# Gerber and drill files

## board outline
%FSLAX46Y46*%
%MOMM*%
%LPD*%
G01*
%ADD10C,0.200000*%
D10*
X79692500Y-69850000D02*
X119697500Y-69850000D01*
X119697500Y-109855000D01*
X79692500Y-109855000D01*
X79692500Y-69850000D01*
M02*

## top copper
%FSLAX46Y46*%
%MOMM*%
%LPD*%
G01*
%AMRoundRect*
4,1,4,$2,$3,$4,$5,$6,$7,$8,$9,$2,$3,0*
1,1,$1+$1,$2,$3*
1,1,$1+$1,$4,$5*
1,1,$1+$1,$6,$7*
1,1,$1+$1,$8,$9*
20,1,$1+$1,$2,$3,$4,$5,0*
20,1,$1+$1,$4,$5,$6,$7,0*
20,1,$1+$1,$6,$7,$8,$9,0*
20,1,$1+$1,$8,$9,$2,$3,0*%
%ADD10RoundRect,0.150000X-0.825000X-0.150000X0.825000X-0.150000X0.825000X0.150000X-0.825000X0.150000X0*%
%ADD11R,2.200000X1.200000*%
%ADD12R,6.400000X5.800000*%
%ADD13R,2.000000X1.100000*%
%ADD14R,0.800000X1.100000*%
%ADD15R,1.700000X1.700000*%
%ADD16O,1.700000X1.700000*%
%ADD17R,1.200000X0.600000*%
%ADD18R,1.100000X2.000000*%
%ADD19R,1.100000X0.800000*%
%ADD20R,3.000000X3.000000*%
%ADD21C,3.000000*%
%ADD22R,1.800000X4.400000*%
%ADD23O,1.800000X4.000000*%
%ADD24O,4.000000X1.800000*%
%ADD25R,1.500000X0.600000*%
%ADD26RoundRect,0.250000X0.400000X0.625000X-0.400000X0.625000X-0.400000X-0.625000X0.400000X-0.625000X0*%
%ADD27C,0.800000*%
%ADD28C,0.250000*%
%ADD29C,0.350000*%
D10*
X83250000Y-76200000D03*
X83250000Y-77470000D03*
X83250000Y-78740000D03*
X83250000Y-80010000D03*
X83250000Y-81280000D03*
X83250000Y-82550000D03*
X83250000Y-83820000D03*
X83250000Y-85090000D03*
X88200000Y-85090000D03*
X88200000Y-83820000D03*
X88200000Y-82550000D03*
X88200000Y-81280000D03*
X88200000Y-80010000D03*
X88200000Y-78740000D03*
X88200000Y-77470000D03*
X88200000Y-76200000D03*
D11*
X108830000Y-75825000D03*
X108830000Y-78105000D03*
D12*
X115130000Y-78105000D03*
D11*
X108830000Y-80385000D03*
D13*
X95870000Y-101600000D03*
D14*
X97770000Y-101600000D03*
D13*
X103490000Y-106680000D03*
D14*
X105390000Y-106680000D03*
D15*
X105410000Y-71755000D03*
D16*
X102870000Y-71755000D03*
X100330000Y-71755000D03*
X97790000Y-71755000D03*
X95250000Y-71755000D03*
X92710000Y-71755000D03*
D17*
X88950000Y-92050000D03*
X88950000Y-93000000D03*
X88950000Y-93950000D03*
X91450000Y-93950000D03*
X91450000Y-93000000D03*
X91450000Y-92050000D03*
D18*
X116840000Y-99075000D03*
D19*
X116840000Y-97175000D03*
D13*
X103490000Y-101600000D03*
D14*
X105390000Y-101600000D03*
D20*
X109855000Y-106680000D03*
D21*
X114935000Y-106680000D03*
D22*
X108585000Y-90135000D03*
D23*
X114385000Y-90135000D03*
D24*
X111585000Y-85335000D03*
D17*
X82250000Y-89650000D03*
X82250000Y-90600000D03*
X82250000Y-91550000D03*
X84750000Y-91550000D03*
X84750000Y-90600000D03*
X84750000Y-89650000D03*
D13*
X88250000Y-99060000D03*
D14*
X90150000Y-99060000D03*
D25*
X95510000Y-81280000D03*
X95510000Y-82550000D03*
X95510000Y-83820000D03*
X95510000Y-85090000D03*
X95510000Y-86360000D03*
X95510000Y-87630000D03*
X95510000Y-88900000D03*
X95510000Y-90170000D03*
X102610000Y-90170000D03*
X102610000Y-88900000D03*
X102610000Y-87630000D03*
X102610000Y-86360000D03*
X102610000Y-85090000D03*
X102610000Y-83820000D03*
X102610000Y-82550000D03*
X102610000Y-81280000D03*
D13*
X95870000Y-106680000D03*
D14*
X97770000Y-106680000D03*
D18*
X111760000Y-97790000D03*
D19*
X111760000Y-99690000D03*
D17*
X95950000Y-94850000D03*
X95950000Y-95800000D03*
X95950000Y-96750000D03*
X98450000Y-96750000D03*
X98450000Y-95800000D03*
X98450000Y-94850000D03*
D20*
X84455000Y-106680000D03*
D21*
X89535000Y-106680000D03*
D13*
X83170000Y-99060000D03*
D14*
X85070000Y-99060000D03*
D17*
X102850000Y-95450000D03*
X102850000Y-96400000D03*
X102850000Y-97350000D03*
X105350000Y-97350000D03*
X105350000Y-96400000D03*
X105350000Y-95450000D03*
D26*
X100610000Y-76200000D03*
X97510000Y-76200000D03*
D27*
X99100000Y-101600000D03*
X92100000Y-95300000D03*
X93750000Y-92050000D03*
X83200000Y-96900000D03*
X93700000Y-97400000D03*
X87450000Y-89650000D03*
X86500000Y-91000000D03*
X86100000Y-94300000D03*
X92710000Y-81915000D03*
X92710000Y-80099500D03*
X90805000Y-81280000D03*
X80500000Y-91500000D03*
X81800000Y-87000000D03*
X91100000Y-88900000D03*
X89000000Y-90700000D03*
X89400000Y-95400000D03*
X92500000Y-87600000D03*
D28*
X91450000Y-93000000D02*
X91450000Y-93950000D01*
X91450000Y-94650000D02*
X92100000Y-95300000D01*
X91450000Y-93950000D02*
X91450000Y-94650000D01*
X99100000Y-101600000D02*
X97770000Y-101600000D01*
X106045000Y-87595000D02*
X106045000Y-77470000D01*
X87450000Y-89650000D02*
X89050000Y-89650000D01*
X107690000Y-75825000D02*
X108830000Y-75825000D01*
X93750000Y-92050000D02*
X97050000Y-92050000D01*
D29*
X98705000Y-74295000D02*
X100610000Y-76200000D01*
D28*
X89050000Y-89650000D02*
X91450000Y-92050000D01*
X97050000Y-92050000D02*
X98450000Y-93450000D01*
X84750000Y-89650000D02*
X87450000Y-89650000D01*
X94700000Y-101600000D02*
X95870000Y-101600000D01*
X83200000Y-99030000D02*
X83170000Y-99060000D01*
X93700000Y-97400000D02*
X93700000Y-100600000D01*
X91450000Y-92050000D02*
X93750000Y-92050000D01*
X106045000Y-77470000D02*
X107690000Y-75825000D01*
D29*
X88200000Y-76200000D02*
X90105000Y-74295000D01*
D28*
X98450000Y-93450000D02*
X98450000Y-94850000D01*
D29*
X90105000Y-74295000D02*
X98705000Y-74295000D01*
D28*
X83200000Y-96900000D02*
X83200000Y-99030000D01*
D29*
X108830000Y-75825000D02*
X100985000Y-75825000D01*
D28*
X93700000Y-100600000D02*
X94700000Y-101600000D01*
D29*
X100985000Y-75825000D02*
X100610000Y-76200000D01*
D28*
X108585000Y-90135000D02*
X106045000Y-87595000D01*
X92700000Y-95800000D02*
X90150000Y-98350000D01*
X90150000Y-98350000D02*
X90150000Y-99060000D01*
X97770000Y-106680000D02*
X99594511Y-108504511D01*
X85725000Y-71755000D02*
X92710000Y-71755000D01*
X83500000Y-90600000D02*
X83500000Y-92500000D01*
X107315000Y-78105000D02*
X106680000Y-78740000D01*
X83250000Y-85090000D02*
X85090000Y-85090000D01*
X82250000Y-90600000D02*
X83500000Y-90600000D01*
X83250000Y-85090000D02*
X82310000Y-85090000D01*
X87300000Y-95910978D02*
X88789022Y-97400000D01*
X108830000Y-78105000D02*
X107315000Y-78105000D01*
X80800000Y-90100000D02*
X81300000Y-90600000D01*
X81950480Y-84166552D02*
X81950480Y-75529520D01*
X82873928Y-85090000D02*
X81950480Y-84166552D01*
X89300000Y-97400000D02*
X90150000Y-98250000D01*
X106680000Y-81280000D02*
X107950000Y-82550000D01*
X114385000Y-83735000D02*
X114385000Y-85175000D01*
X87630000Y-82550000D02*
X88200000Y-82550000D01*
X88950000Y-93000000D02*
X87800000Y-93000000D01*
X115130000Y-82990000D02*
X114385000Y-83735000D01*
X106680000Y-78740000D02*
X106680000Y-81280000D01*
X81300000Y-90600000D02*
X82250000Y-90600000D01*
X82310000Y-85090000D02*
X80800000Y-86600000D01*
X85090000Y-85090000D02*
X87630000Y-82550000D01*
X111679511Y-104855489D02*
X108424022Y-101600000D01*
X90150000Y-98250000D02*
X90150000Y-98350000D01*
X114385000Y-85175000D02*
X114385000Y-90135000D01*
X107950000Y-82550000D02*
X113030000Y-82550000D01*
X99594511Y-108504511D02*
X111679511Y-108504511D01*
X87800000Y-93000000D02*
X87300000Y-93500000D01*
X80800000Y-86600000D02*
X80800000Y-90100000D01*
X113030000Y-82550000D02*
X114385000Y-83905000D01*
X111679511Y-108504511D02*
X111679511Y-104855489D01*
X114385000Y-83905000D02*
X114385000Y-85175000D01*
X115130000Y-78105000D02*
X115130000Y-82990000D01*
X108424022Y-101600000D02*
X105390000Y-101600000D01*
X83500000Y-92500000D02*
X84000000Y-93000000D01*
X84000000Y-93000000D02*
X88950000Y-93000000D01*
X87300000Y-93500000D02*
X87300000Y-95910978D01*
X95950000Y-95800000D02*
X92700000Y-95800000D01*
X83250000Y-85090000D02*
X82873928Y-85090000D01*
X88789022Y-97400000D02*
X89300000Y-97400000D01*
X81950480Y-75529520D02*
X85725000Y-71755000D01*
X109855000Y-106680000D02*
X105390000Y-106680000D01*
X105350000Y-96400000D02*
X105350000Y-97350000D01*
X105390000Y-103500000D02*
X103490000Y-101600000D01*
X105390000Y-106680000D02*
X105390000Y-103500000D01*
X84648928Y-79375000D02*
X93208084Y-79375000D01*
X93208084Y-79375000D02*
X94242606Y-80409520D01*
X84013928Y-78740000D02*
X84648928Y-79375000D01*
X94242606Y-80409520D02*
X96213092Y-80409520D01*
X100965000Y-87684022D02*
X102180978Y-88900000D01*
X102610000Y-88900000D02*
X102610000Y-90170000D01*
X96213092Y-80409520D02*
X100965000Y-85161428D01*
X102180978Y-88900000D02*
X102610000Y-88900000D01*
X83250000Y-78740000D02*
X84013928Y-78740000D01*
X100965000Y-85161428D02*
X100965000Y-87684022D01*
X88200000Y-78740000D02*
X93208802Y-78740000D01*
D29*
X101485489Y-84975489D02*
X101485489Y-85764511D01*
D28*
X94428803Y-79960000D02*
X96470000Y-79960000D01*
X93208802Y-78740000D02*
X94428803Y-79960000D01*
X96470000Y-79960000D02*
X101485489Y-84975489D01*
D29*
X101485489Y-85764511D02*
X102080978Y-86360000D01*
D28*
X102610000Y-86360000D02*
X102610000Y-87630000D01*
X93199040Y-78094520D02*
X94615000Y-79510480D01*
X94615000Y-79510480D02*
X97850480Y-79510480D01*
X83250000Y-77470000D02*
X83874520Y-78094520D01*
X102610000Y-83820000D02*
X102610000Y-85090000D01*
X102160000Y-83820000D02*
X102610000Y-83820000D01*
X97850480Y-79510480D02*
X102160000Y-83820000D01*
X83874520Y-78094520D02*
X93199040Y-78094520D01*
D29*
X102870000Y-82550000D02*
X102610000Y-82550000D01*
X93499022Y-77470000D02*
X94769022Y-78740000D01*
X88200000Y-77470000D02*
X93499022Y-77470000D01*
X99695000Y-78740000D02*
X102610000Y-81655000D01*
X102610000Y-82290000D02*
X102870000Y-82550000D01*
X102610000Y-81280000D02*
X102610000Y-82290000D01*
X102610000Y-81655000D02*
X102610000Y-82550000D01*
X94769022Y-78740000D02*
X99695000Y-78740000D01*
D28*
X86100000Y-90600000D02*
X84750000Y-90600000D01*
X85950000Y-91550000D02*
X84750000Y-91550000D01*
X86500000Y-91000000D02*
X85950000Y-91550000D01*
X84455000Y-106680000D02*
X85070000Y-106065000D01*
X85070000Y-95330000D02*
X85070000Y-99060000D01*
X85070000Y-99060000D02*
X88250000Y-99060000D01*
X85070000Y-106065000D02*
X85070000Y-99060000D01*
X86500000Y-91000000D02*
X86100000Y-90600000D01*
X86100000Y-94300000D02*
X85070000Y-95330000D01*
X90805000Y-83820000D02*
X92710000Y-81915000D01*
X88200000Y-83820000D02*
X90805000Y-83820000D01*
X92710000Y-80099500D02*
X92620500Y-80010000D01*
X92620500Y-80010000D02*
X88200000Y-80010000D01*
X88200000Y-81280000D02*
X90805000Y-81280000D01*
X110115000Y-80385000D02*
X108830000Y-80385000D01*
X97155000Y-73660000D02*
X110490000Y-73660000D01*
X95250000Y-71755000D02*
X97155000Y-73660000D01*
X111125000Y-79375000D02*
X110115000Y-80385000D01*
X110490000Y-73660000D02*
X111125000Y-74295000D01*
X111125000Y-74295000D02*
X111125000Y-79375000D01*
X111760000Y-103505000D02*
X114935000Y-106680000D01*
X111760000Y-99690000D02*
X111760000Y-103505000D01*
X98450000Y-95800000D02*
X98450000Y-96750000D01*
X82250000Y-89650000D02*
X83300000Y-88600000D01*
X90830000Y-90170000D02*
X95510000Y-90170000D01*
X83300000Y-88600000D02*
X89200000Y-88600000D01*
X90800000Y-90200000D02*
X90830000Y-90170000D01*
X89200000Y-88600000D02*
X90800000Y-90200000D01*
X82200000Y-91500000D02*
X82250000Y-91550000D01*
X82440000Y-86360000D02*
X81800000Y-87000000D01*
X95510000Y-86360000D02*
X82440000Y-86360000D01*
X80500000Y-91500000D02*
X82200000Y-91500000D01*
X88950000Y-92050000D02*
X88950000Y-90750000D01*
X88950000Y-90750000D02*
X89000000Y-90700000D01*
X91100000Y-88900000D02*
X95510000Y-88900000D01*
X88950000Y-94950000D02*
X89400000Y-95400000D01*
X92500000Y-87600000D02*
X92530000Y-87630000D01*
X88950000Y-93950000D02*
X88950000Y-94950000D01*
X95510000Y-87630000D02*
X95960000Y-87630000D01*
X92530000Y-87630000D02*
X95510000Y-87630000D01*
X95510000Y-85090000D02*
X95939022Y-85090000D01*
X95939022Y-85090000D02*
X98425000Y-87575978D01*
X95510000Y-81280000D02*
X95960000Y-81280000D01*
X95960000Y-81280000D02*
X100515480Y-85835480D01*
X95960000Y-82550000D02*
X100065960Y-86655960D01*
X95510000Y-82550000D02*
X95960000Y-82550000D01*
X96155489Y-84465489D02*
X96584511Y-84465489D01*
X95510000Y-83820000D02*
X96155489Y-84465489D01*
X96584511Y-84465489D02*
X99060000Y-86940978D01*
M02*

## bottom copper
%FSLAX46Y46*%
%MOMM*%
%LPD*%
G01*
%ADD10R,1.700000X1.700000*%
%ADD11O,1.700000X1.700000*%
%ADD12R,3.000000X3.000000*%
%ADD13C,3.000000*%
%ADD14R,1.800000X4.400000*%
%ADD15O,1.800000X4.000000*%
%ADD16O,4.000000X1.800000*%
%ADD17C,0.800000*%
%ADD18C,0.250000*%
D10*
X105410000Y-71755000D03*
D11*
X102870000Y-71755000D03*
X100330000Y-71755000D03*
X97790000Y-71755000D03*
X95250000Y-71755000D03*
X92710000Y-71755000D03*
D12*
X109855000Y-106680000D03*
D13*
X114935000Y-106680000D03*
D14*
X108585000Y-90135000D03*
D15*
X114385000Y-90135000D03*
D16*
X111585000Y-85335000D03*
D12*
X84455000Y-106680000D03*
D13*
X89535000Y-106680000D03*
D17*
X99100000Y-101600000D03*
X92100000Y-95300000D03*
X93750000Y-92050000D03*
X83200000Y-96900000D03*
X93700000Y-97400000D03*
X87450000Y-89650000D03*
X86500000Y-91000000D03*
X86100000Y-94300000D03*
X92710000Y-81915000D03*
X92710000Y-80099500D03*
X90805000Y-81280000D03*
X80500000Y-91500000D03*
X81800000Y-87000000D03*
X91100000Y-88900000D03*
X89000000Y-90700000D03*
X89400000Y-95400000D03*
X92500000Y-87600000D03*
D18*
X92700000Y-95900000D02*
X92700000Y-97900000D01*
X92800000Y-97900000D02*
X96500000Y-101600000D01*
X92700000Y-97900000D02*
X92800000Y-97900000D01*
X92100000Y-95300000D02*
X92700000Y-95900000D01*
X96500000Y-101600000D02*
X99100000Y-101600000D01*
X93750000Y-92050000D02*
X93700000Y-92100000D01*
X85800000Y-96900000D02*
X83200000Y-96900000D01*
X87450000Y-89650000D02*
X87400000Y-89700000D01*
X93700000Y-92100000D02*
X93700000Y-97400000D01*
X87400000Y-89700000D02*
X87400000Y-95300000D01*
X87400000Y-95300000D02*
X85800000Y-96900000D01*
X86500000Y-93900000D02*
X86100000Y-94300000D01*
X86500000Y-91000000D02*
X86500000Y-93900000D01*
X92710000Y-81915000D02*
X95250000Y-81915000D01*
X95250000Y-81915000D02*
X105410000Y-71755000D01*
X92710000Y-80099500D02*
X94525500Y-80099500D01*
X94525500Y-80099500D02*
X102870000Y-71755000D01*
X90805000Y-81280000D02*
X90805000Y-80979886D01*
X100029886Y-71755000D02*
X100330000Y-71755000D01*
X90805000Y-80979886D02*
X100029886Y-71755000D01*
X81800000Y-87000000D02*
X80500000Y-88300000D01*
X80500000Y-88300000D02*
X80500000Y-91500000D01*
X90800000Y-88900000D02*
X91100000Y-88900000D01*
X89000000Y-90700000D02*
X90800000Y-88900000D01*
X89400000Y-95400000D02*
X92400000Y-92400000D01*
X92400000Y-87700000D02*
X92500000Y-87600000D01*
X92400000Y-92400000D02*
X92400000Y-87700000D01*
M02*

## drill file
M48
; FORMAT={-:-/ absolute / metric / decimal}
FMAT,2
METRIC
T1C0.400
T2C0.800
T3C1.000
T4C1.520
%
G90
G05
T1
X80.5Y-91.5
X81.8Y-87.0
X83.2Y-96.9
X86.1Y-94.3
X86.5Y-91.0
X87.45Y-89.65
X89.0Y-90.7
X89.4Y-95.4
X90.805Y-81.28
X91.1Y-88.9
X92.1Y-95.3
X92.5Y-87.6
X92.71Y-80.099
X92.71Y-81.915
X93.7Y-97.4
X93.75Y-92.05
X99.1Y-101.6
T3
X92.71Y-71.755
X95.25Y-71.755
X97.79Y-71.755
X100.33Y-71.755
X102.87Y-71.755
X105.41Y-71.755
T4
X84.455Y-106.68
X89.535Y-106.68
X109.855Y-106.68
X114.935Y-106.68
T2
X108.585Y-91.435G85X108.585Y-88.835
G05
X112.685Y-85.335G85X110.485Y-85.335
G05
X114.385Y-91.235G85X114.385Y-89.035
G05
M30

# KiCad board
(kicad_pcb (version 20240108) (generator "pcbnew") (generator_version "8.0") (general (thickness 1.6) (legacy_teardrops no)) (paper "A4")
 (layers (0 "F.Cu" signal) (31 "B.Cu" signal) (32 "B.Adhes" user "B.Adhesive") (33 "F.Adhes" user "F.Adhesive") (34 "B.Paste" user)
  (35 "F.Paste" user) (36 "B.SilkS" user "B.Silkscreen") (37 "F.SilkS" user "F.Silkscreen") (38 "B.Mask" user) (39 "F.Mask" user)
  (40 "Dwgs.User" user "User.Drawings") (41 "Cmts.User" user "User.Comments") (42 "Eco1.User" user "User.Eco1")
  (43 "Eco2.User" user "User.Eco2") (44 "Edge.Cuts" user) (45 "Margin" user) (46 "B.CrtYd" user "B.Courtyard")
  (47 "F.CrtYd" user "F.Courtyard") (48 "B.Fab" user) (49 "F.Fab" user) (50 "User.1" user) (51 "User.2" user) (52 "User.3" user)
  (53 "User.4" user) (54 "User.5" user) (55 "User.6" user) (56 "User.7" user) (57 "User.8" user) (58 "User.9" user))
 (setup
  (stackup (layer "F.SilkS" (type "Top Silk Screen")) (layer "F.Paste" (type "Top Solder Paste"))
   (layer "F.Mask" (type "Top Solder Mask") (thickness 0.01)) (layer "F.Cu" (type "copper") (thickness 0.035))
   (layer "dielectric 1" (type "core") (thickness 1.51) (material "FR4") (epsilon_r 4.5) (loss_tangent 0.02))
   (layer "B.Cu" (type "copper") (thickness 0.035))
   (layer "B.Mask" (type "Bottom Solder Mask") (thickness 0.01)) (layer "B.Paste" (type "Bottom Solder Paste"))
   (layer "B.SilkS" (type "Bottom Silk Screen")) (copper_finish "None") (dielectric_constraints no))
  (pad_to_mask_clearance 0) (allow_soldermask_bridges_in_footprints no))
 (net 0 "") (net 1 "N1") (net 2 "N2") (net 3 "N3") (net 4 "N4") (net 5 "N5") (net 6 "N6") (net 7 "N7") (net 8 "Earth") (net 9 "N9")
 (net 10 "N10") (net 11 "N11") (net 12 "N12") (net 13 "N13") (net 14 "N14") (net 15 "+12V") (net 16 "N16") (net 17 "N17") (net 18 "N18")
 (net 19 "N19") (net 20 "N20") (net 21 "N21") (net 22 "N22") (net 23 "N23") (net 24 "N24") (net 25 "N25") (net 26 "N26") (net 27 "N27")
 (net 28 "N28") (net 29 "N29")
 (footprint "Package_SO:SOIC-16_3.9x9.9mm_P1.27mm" (layer "F.Cu") (at 85.725 80.645)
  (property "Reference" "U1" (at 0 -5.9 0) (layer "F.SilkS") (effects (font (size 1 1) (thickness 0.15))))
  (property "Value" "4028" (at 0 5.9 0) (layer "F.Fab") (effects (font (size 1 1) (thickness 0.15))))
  (pad "1" smd roundrect (at -2.475 -4.445) (size 1.95 0.6) (layers "F.Cu" "F.Paste" "F.Mask") (roundrect_rratio 0.25) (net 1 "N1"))
  (pad "2" smd roundrect (at -2.475 -3.175) (size 1.95 0.6) (layers "F.Cu" "F.Paste" "F.Mask") (roundrect_rratio 0.25) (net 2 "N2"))
  (pad "3" smd roundrect (at -2.475 -1.905) (size 1.95 0.6) (layers "F.Cu" "F.Paste" "F.Mask") (roundrect_rratio 0.25) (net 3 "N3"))
  (pad "4" smd roundrect (at -2.475 -0.635) (size 1.95 0.6) (layers "F.Cu" "F.Paste" "F.Mask") (roundrect_rratio 0.25) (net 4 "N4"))
  (pad "5" smd roundrect (at -2.475 0.635) (size 1.95 0.6) (layers "F.Cu" "F.Paste" "F.Mask") (roundrect_rratio 0.25) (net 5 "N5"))
  (pad "6" smd roundrect (at -2.475 1.905) (size 1.95 0.6) (layers "F.Cu" "F.Paste" "F.Mask") (roundrect_rratio 0.25) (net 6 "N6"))
  (pad "7" smd roundrect (at -2.475 3.175) (size 1.95 0.6) (layers "F.Cu" "F.Paste" "F.Mask") (roundrect_rratio 0.25) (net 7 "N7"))
  (pad "8" smd roundrect (at -2.475 4.445) (size 1.95 0.6) (layers "F.Cu" "F.Paste" "F.Mask") (roundrect_rratio 0.25) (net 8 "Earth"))
  (pad "9" smd roundrect (at 2.475 4.445) (size 1.95 0.6) (layers "F.Cu" "F.Paste" "F.Mask") (roundrect_rratio 0.25) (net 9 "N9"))
  (pad "10" smd roundrect (at 2.475 3.175) (size 1.95 0.6) (layers "F.Cu" "F.Paste" "F.Mask") (roundrect_rratio 0.25) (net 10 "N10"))
  (pad "11" smd roundrect (at 2.475 1.905) (size 1.95 0.6) (layers "F.Cu" "F.Paste" "F.Mask") (roundrect_rratio 0.25) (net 8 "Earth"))
  (pad "12" smd roundrect (at 2.475 0.635) (size 1.95 0.6) (layers "F.Cu" "F.Paste" "F.Mask") (roundrect_rratio 0.25) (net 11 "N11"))
  (pad "13" smd roundrect (at 2.475 -0.635) (size 1.95 0.6) (layers "F.Cu" "F.Paste" "F.Mask") (roundrect_rratio 0.25) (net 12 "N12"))
  (pad "14" smd roundrect (at 2.475 -1.905) (size 1.95 0.6) (layers "F.Cu" "F.Paste" "F.Mask") (roundrect_rratio 0.25) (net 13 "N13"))
  (pad "15" smd roundrect (at 2.475 -3.175) (size 1.95 0.6) (layers "F.Cu" "F.Paste" "F.Mask") (roundrect_rratio 0.25) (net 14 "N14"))
  (pad "16" smd roundrect (at 2.475 -4.445) (size 1.95 0.6) (layers "F.Cu" "F.Paste" "F.Mask") (roundrect_rratio 0.25) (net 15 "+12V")))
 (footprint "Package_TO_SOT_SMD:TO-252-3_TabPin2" (layer "F.Cu") (at 113.03 78.105)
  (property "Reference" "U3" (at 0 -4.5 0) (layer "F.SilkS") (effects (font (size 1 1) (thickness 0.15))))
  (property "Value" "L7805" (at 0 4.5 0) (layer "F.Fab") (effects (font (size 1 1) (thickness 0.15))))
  (pad "" smd rect (at 0.425 -1.525) (size 3.05 2.75) (layers "F.Paste"))
  (pad "" smd rect (at 0.425 1.525) (size 3.05 2.75) (layers "F.Paste"))
  (pad "" smd rect (at 3.775 -1.525) (size 3.05 2.75) (layers "F.Paste"))
  (pad "" smd rect (at 3.775 1.525) (size 3.05 2.75) (layers "F.Paste"))
  (pad "1" smd rect (at -4.2 -2.28) (size 2.2 1.2) (layers "F.Cu" "F.Paste" "F.Mask") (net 15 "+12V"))
  (pad "2" smd rect (at -4.2 0) (size 2.2 1.2) (layers "F.Cu" "F.Paste" "F.Mask") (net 8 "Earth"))
  (pad "2" smd rect (at 2.1 0) (size 6.4 5.8) (layers "F.Cu" "F.Mask") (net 8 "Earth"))
  (pad "3" smd rect (at -4.2 2.28) (size 2.2 1.2) (layers "F.Cu" "F.Paste" "F.Mask") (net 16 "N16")))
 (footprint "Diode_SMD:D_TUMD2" (layer "F.Cu") (at 96.52 101.6)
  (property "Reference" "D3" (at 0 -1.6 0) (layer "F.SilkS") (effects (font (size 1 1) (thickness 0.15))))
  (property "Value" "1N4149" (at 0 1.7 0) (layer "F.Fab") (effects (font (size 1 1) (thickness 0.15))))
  (pad "1" smd rect (at -0.65 0 180) (size 2 1.1) (layers "F.Cu" "F.Paste" "F.Mask") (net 15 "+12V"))
  (pad "2" smd rect (at 1.25 0 180) (size 0.8 1.1) (layers "F.Cu" "F.Paste" "F.Mask") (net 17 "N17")))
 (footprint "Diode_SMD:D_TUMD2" (layer "F.Cu") (at 104.14 106.68)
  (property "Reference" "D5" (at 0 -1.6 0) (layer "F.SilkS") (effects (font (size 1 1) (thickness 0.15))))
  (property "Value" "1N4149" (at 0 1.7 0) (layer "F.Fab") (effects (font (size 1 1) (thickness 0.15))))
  (pad "1" smd rect (at -0.65 0 180) (size 2 1.1) (layers "F.Cu" "F.Paste" "F.Mask") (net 15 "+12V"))
  (pad "2" smd rect (at 1.25 0 180) (size 0.8 1.1) (layers "F.Cu" "F.Paste" "F.Mask") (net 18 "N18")))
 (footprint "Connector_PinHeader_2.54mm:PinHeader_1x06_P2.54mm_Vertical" (layer "F.Cu") (at 105.41 71.755 -90)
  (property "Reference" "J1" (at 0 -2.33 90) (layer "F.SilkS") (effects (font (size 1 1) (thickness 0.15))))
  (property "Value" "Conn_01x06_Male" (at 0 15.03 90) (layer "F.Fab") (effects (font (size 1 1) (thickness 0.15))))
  (pad "1" thru_hole rect (at 0 0 270) (size 1.7 1.7) (drill 1) (layers "*.Cu" "*.Mask") (remove_unused_layers no) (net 10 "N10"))
  (pad "2" thru_hole oval (at 0 2.54 270) (size 1.7 1.7) (drill 1) (layers "*.Cu" "*.Mask") (remove_unused_layers no) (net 12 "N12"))
  (pad "3" thru_hole oval (at 0 5.08 270) (size 1.7 1.7) (drill 1) (layers "*.Cu" "*.Mask") (remove_unused_layers no) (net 11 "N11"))
  (pad "4" thru_hole oval (at 0 7.62 270) (size 1.7 1.7) (drill 1) (layers "*.Cu" "*.Mask") (remove_unused_layers no) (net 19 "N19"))
  (pad "5" thru_hole oval (at 0 10.16 270) (size 1.7 1.7) (drill 1) (layers "*.Cu" "*.Mask") (remove_unused_layers no) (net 16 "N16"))
  (pad "6" thru_hole oval (at 0 12.7 270) (size 1.7 1.7) (drill 1) (layers "*.Cu" "*.Mask") (remove_unused_layers no) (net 8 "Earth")))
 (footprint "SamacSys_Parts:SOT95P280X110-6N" (layer "F.Cu") (at 90.2 93)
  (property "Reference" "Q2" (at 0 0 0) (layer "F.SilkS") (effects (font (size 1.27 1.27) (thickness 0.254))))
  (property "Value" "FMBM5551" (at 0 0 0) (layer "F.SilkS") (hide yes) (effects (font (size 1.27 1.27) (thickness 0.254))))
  (pad "1" smd rect (at -1.25 -0.95 90) (size 0.6 1.2) (layers "F.Cu" "F.Paste" "F.Mask") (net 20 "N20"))
  (pad "2" smd rect (at -1.25 0 90) (size 0.6 1.2) (layers "F.Cu" "F.Paste" "F.Mask") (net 8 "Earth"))
  (pad "3" smd rect (at -1.25 0.95 90) (size 0.6 1.2) (layers "F.Cu" "F.Paste" "F.Mask") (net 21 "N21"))
  (pad "4" smd rect (at 1.25 0.95 90) (size 0.6 1.2) (layers "F.Cu" "F.Paste" "F.Mask") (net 17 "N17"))
  (pad "5" smd rect (at 1.25 0 90) (size 0.6 1.2) (layers "F.Cu" "F.Paste" "F.Mask") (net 17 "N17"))
  (pad "6" smd rect (at 1.25 -0.95 90) (size 0.6 1.2) (layers "F.Cu" "F.Paste" "F.Mask") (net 15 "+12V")))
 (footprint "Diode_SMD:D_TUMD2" (layer "F.Cu") (at 116.84 98.425 90)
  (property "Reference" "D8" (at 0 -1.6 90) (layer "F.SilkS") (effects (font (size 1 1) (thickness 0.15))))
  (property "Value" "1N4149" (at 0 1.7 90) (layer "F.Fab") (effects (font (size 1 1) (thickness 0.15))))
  (pad "1" smd rect (at -0.65 0 270) (size 2 1.1) (layers "F.Cu" "F.Paste" "F.Mask") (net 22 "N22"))
  (pad "2" smd rect (at 1.25 0 270) (size 0.8 1.1) (layers "F.Cu" "F.Paste" "F.Mask") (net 8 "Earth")))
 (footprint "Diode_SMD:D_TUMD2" (layer "F.Cu") (at 104.14 101.6)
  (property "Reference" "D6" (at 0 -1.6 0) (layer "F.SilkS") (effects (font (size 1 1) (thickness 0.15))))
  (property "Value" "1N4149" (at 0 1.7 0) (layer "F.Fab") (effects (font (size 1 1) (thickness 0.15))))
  (pad "1" smd rect (at -0.65 0 180) (size 2 1.1) (layers "F.Cu" "F.Paste" "F.Mask") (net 18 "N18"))
  (pad "2" smd rect (at 1.25 0 180) (size 0.8 1.1) (layers "F.Cu" "F.Paste" "F.Mask") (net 8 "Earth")))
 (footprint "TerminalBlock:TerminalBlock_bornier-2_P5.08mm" (layer "F.Cu") (at 109.855 106.68)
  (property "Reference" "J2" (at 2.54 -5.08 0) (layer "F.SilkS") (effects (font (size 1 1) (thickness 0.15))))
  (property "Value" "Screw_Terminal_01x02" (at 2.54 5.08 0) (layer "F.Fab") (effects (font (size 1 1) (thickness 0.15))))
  (pad "1" thru_hole rect (at 0 0) (size 3 3) (drill 1.52) (layers "*.Cu" "*.Mask") (remove_unused_layers no) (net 18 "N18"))
  (pad "2" thru_hole circle (at 5.08 0) (size 3 3) (drill 1.52) (layers "*.Cu" "*.Mask") (remove_unused_layers no) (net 22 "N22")))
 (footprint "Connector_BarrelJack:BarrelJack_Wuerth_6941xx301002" (layer "F.Cu") (at 108.585 90.135 90)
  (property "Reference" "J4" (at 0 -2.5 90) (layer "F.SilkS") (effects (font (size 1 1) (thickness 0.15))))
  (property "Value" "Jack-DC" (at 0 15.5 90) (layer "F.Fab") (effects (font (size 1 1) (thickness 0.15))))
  (pad "1" thru_hole rect (at 0 0 90) (size 4.4 1.8) (drill oval 3.4 0.8) (layers "*.Cu" "*.Mask") (remove_unused_layers no) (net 15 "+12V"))
  (pad "2" thru_hole oval (at 0 5.8 90) (size 4 1.8) (drill oval 3 0.8) (layers "*.Cu" "*.Mask") (remove_unused_layers no) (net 8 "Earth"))
  (pad "3" thru_hole oval (at 4.8 3 180) (size 4 1.8) (drill oval 3 0.8) (layers "*.Cu" "*.Mask") (remove_unused_layers no)))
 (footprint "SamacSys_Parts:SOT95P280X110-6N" (layer "F.Cu") (at 83.5 90.6)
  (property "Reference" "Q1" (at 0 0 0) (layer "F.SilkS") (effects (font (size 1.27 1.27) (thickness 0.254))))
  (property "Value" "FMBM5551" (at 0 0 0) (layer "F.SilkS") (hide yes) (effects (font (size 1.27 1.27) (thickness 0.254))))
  (pad "1" smd rect (at -1.25 -0.95 90) (size 0.6 1.2) (layers "F.Cu" "F.Paste" "F.Mask") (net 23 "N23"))
  (pad "2" smd rect (at -1.25 0 90) (size 0.6 1.2) (layers "F.Cu" "F.Paste" "F.Mask") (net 8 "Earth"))
  (pad "3" smd rect (at -1.25 0.95 90) (size 0.6 1.2) (layers "F.Cu" "F.Paste" "F.Mask") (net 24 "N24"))
  (pad "4" smd rect (at 1.25 0.95 90) (size 0.6 1.2) (layers "F.Cu" "F.Paste" "F.Mask") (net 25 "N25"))
  (pad "5" smd rect (at 1.25 0 90) (size 0.6 1.2) (layers "F.Cu" "F.Paste" "F.Mask") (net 25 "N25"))
  (pad "6" smd rect (at 1.25 -0.95 90) (size 0.6 1.2) (layers "F.Cu" "F.Paste" "F.Mask") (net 15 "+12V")))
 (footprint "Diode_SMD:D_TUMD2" (layer "F.Cu") (at 88.9 99.06)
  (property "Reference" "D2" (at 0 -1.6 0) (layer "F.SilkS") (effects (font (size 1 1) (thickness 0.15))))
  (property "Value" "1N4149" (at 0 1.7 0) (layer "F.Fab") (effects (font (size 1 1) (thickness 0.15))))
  (pad "1" smd rect (at -0.65 0 180) (size 2 1.1) (layers "F.Cu" "F.Paste" "F.Mask") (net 25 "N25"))
  (pad "2" smd rect (at 1.25 0 180) (size 0.8 1.1) (layers "F.Cu" "F.Paste" "F.Mask") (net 8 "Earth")))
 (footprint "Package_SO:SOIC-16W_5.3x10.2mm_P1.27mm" (layer "F.Cu") (at 99.06 85.725)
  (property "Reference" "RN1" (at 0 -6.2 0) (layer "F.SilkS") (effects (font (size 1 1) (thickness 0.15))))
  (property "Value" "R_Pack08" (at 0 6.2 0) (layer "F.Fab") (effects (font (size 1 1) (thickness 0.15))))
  (pad "1" smd rect (at -3.55 -4.445) (size 1.5 0.6) (layers "F.Cu" "F.Paste" "F.Mask") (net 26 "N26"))
  (pad "2" smd rect (at -3.55 -3.175) (size 1.5 0.6) (layers "F.Cu" "F.Paste" "F.Mask") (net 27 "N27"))
  (pad "3" smd rect (at -3.55 -1.905) (size 1.5 0.6) (layers "F.Cu" "F.Paste" "F.Mask") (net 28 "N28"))
  (pad "4" smd rect (at -3.55 -0.635) (size 1.5 0.6) (layers "F.Cu" "F.Paste" "F.Mask") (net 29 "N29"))
  (pad "5" smd rect (at -3.55 0.635) (size 1.5 0.6) (layers "F.Cu" "F.Paste" "F.Mask") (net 24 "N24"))
  (pad "6" smd rect (at -3.55 1.905) (size 1.5 0.6) (layers "F.Cu" "F.Paste" "F.Mask") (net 21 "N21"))
  (pad "7" smd rect (at -3.55 3.175) (size 1.5 0.6) (layers "F.Cu" "F.Paste" "F.Mask") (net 20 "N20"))
  (pad "8" smd rect (at -3.55 4.445) (size 1.5 0.6) (layers "F.Cu" "F.Paste" "F.Mask") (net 23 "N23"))
  (pad "9" smd rect (at 3.55 4.445) (size 1.5 0.6) (layers "F.Cu" "F.Paste" "F.Mask") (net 3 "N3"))
  (pad "10" smd rect (at 3.55 3.175) (size 1.5 0.6) (layers "F.Cu" "F.Paste" "F.Mask") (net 3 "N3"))
  (pad "11" smd rect (at 3.55 1.905) (size 1.5 0.6) (layers "F.Cu" "F.Paste" "F.Mask") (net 13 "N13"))
  (pad "12" smd rect (at 3.55 0.635) (size 1.5 0.6) (layers "F.Cu" "F.Paste" "F.Mask") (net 13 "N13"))
  (pad "13" smd rect (at 3.55 -0.635) (size 1.5 0.6) (layers "F.Cu" "F.Paste" "F.Mask") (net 2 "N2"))
  (pad "14" smd rect (at 3.55 -1.905) (size 1.5 0.6) (layers "F.Cu" "F.Paste" "F.Mask") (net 2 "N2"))
  (pad "15" smd rect (at 3.55 -3.175) (size 1.5 0.6) (layers "F.Cu" "F.Paste" "F.Mask") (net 14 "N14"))
  (pad "16" smd rect (at 3.55 -4.445) (size 1.5 0.6) (layers "F.Cu" "F.Paste" "F.Mask") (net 14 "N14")))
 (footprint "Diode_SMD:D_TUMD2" (layer "F.Cu") (at 96.52 106.68)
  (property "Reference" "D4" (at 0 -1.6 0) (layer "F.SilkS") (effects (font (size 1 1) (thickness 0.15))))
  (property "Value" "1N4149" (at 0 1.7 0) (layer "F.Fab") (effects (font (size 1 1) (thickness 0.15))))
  (pad "1" smd rect (at -0.65 0 180) (size 2 1.1) (layers "F.Cu" "F.Paste" "F.Mask") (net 17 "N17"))
  (pad "2" smd rect (at 1.25 0 180) (size 0.8 1.1) (layers "F.Cu" "F.Paste" "F.Mask") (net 8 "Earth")))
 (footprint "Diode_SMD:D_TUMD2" (layer "F.Cu") (at 111.76 98.44 -90)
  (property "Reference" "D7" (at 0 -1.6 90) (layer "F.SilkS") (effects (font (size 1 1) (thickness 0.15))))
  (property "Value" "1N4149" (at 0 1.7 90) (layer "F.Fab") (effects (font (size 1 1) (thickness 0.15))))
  (pad "1" smd rect (at -0.65 0 90) (size 2 1.1) (layers "F.Cu" "F.Paste" "F.Mask") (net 15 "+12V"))
  (pad "2" smd rect (at 1.25 0 90) (size 0.8 1.1) (layers "F.Cu" "F.Paste" "F.Mask") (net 22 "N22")))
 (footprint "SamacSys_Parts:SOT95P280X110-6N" (layer "F.Cu") (at 97.2 95.8)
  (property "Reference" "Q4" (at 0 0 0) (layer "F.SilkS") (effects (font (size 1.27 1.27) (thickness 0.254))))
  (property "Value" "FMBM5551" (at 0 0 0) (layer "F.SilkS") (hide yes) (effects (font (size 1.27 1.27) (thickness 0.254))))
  (pad "1" smd rect (at -1.25 -0.95 90) (size 0.6 1.2) (layers "F.Cu" "F.Paste" "F.Mask") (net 27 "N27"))
  (pad "2" smd rect (at -1.25 0 90) (size 0.6 1.2) (layers "F.Cu" "F.Paste" "F.Mask") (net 8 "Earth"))
  (pad "3" smd rect (at -1.25 0.95 90) (size 0.6 1.2) (layers "F.Cu" "F.Paste" "F.Mask") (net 28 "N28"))
  (pad "4" smd rect (at 1.25 0.95 90) (size 0.6 1.2) (layers "F.Cu" "F.Paste" "F.Mask") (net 22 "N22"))
  (pad "5" smd rect (at 1.25 0 90) (size 0.6 1.2) (layers "F.Cu" "F.Paste" "F.Mask") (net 22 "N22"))
  (pad "6" smd rect (at 1.25 -0.95 90) (size 0.6 1.2) (layers "F.Cu" "F.Paste" "F.Mask") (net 15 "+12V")))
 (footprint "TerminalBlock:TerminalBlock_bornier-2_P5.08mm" (layer "F.Cu") (at 84.455 106.68)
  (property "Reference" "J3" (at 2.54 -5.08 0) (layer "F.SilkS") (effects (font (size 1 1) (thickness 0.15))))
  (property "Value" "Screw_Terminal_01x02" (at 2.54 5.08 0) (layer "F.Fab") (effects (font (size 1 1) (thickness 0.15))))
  (pad "1" thru_hole rect (at 0 0) (size 3 3) (drill 1.52) (layers "*.Cu" "*.Mask") (remove_unused_layers no) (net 25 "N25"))
  (pad "2" thru_hole circle (at 5.08 0) (size 3 3) (drill 1.52) (layers "*.Cu" "*.Mask") (remove_unused_layers no) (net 17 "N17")))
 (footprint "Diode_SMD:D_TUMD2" (layer "F.Cu") (at 83.82 99.06)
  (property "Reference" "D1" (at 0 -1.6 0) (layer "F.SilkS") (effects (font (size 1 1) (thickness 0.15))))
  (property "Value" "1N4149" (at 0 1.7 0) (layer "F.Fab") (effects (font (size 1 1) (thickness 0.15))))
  (pad "1" smd rect (at -0.65 0 180) (size 2 1.1) (layers "F.Cu" "F.Paste" "F.Mask") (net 15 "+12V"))
  (pad "2" smd rect (at 1.25 0 180) (size 0.8 1.1) (layers "F.Cu" "F.Paste" "F.Mask") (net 25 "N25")))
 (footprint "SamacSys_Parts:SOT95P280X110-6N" (layer "F.Cu") (at 104.1 96.4)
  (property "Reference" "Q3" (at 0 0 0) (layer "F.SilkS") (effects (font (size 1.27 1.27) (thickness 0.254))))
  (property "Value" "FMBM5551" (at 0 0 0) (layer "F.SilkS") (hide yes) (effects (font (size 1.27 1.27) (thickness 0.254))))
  (pad "1" smd rect (at -1.25 -0.95 90) (size 0.6 1.2) (layers "F.Cu" "F.Paste" "F.Mask") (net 29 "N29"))
  (pad "2" smd rect (at -1.25 0 90) (size 0.6 1.2) (layers "F.Cu" "F.Paste" "F.Mask") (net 8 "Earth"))
  (pad "3" smd rect (at -1.25 0.95 90) (size 0.6 1.2) (layers "F.Cu" "F.Paste" "F.Mask") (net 26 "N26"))
  (pad "4" smd rect (at 1.25 0.95 90) (size 0.6 1.2) (layers "F.Cu" "F.Paste" "F.Mask") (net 18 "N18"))
  (pad "5" smd rect (at 1.25 0 90) (size 0.6 1.2) (layers "F.Cu" "F.Paste" "F.Mask") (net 18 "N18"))
  (pad "6" smd rect (at 1.25 -0.95 90) (size 0.6 1.2) (layers "F.Cu" "F.Paste" "F.Mask") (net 15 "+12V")))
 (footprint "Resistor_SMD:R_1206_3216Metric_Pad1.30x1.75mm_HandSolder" (layer "F.Cu") (at 99.06 76.2 180)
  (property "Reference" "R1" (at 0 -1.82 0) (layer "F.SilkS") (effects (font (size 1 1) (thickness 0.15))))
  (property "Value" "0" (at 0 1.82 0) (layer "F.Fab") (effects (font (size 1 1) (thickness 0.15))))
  (pad "1" smd roundrect (at -1.55 0 180) (size 1.3 1.75) (layers "F.Cu" "F.Paste" "F.Mask") (roundrect_rratio 0.192308) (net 15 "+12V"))
  (pad "2" smd roundrect (at 1.55 0 180) (size 1.3 1.75) (layers "F.Cu" "F.Paste" "F.Mask") (roundrect_rratio 0.192308) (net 19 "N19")))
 (gr_rect (start 79.6925 69.85) (end 119.6975 109.855) (stroke (width 0.2) (type solid)) (fill none) (layer "Edge.Cuts"))
 (segment (start 91.45 93) (end 91.45 93.95) (width 0.25) (layer "F.Cu") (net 17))
 (segment (start 91.45 94.65) (end 92.1 95.3) (width 0.25) (layer "F.Cu") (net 17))
 (segment (start 91.45 93.95) (end 91.45 94.65) (width 0.25) (layer "F.Cu") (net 17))
 (segment (start 99.1 101.6) (end 97.77 101.6) (width 0.25) (layer "F.Cu") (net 17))
 (via (at 99.1 101.6) (size 0.8) (drill 0.4) (layers "F.Cu" "B.Cu") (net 17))
 (via (at 92.1 95.3) (size 0.8) (drill 0.4) (layers "F.Cu" "B.Cu") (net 17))
 (segment (start 92.7 95.9) (end 92.7 97.9) (width 0.25) (layer "B.Cu") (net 17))
 (segment (start 92.8 97.9) (end 96.5 101.6) (width 0.25) (layer "B.Cu") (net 17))
 (segment (start 92.7 97.9) (end 92.8 97.9) (width 0.25) (layer "B.Cu") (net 17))
 (segment (start 92.1 95.3) (end 92.7 95.9) (width 0.25) (layer "B.Cu") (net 17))
 (segment (start 96.5 101.6) (end 99.1 101.6) (width 0.25) (layer "B.Cu") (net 17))
 (segment (start 106.045 87.595) (end 106.045 77.47) (width 0.25) (layer "F.Cu") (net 15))
 (segment (start 87.45 89.65) (end 89.05 89.65) (width 0.25) (layer "F.Cu") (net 15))
 (segment (start 107.69 75.825) (end 108.83 75.825) (width 0.25) (layer "F.Cu") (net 15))
 (segment (start 93.75 92.05) (end 97.05 92.05) (width 0.25) (layer "F.Cu") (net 15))
 (segment (start 98.705 74.295) (end 100.61 76.2) (width 0.35) (layer "F.Cu") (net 15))
 (segment (start 89.05 89.65) (end 91.45 92.05) (width 0.25) (layer "F.Cu") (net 15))
 (segment (start 97.05 92.05) (end 98.45 93.45) (width 0.25) (layer "F.Cu") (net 15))
 (segment (start 84.75 89.65) (end 87.45 89.65) (width 0.25) (layer "F.Cu") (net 15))
 (segment (start 94.7 101.6) (end 95.87 101.6) (width 0.25) (layer "F.Cu") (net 15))
 (segment (start 83.2 99.03) (end 83.17 99.06) (width 0.25) (layer "F.Cu") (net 15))
 (segment (start 93.7 97.4) (end 93.7 100.6) (width 0.25) (layer "F.Cu") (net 15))
 (segment (start 91.45 92.05) (end 93.75 92.05) (width 0.25) (layer "F.Cu") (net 15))
 (segment (start 106.045 77.47) (end 107.69 75.825) (width 0.25) (layer "F.Cu") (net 15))
 (segment (start 88.2 76.2) (end 90.105 74.295) (width 0.35) (layer "F.Cu") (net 15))
 (segment (start 98.45 93.45) (end 98.45 94.85) (width 0.25) (layer "F.Cu") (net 15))
 (segment (start 90.105 74.295) (end 98.705 74.295) (width 0.35) (layer "F.Cu") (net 15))
 (segment (start 83.2 96.9) (end 83.2 99.03) (width 0.25) (layer "F.Cu") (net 15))
 (segment (start 108.83 75.825) (end 100.985 75.825) (width 0.35) (layer "F.Cu") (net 15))
 (segment (start 93.7 100.6) (end 94.7 101.6) (width 0.25) (layer "F.Cu") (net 15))
 (segment (start 100.985 75.825) (end 100.61 76.2) (width 0.35) (layer "F.Cu") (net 15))
 (segment (start 108.585 90.135) (end 106.045 87.595) (width 0.25) (layer "F.Cu") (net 15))
 (via (at 93.75 92.05) (size 0.8) (drill 0.4) (layers "F.Cu" "B.Cu") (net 15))
 (via (at 83.2 96.9) (size 0.8) (drill 0.4) (layers "F.Cu" "B.Cu") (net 15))
 (via (at 93.7 97.4) (size 0.8) (drill 0.4) (layers "F.Cu" "B.Cu") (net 15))
 (via (at 87.45 89.65) (size 0.8) (drill 0.4) (layers "F.Cu" "B.Cu") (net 15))
 (segment (start 93.75 92.05) (end 93.7 92.1) (width 0.25) (layer "B.Cu") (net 15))
 (segment (start 85.8 96.9) (end 83.2 96.9) (width 0.25) (layer "B.Cu") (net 15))
 (segment (start 87.45 89.65) (end 87.4 89.7) (width 0.25) (layer "B.Cu") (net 15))
 (segment (start 93.7 92.1) (end 93.7 97.4) (width 0.25) (layer "B.Cu") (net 15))
 (segment (start 87.4 89.7) (end 87.4 95.3) (width 0.25) (layer "B.Cu") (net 15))
 (segment (start 87.4 95.3) (end 85.8 96.9) (width 0.25) (layer "B.Cu") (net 15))
 (segment (start 92.7 95.8) (end 90.15 98.35) (width 0.25) (layer "F.Cu") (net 8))
 (segment (start 90.15 98.35) (end 90.15 99.06) (width 0.25) (layer "F.Cu") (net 8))
 (segment (start 97.77 106.68) (end 99.594511 108.504511) (width 0.25) (layer "F.Cu") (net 8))
 (segment (start 85.725 71.755) (end 92.71 71.755) (width 0.25) (layer "F.Cu") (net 8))
 (segment (start 83.5 90.6) (end 83.5 92.5) (width 0.25) (layer "F.Cu") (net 8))
 (segment (start 107.315 78.105) (end 106.68 78.74) (width 0.25) (layer "F.Cu") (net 8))
 (segment (start 83.25 85.09) (end 85.09 85.09) (width 0.25) (layer "F.Cu") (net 8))
 (segment (start 82.25 90.6) (end 83.5 90.6) (width 0.25) (layer "F.Cu") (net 8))
 (segment (start 83.25 85.09) (end 82.31 85.09) (width 0.25) (layer "F.Cu") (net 8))
 (segment (start 87.3 95.910978) (end 88.789022 97.4) (width 0.25) (layer "F.Cu") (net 8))
 (segment (start 108.83 78.105) (end 107.315 78.105) (width 0.25) (layer "F.Cu") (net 8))
 (segment (start 80.8 90.1) (end 81.3 90.6) (width 0.25) (layer "F.Cu") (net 8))
 (segment (start 81.95048 84.166552) (end 81.95048 75.52952) (width 0.25) (layer "F.Cu") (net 8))
 (segment (start 82.873928 85.09) (end 81.95048 84.166552) (width 0.25) (layer "F.Cu") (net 8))
 (segment (start 89.3 97.4) (end 90.15 98.25) (width 0.25) (layer "F.Cu") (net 8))
 (segment (start 106.68 81.28) (end 107.95 82.55) (width 0.25) (layer "F.Cu") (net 8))
 (segment (start 114.385 83.735) (end 114.385 85.175) (width 0.25) (layer "F.Cu") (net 8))
 (segment (start 87.63 82.55) (end 88.2 82.55) (width 0.25) (layer "F.Cu") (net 8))
 (segment (start 88.95 93) (end 87.8 93) (width 0.25) (layer "F.Cu") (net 8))
 (segment (start 115.13 82.99) (end 114.385 83.735) (width 0.25) (layer "F.Cu") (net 8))
 (segment (start 106.68 78.74) (end 106.68 81.28) (width 0.25) (layer "F.Cu") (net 8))
 (segment (start 81.3 90.6) (end 82.25 90.6) (width 0.25) (layer "F.Cu") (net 8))
 (segment (start 82.31 85.09) (end 80.8 86.6) (width 0.25) (layer "F.Cu") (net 8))
 (segment (start 85.09 85.09) (end 87.63 82.55) (width 0.25) (layer "F.Cu") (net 8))
 (segment (start 111.679511 104.855489) (end 108.424022 101.6) (width 0.25) (layer "F.Cu") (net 8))
 (segment (start 90.15 98.25) (end 90.15 98.35) (width 0.25) (layer "F.Cu") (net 8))
 (segment (start 114.385 85.175) (end 114.385 90.135) (width 0.25) (layer "F.Cu") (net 8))
 (segment (start 107.95 82.55) (end 113.03 82.55) (width 0.25) (layer "F.Cu") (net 8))
 (segment (start 99.594511 108.504511) (end 111.679511 108.504511) (width 0.25) (layer "F.Cu") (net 8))
 (segment (start 87.8 93) (end 87.3 93.5) (width 0.25) (layer "F.Cu") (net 8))
 (segment (start 80.8 86.6) (end 80.8 90.1) (width 0.25) (layer "F.Cu") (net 8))
 (segment (start 113.03 82.55) (end 114.385 83.905) (width 0.25) (layer "F.Cu") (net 8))
 (segment (start 111.679511 108.504511) (end 111.679511 104.855489) (width 0.25) (layer "F.Cu") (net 8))
 (segment (start 114.385 83.905) (end 114.385 85.175) (width 0.25) (layer "F.Cu") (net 8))
 (segment (start 115.13 78.105) (end 115.13 82.99) (width 0.25) (layer "F.Cu") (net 8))
 (segment (start 108.424022 101.6) (end 105.39 101.6) (width 0.25) (layer "F.Cu") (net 8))
 (segment (start 83.5 92.5) (end 84 93) (width 0.25) (layer "F.Cu") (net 8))
 (segment (start 84 93) (end 88.95 93) (width 0.25) (layer "F.Cu") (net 8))
 (segment (start 87.3 93.5) (end 87.3 95.910978) (width 0.25) (layer "F.Cu") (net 8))
 (segment (start 95.95 95.8) (end 92.7 95.8) (width 0.25) (layer "F.Cu") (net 8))
 (segment (start 83.25 85.09) (end 82.873928 85.09) (width 0.25) (layer "F.Cu") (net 8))
 (segment (start 88.789022 97.4) (end 89.3 97.4) (width 0.25) (layer "F.Cu") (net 8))
 (segment (start 81.95048 75.52952) (end 85.725 71.755) (width 0.25) (layer "F.Cu") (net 8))
 (segment (start 109.855 106.68) (end 105.39 106.68) (width 0.25) (layer "F.Cu") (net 18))
 (segment (start 105.35 96.4) (end 105.35 97.35) (width 0.25) (layer "F.Cu") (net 18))
 (segment (start 105.39 103.5) (end 103.49 101.6) (width 0.25) (layer "F.Cu") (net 18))
 (segment (start 105.39 106.68) (end 105.39 103.5) (width 0.25) (layer "F.Cu") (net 18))
 (segment (start 84.648928 79.375) (end 93.208084 79.375) (width 0.25) (layer "F.Cu") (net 3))
 (segment (start 93.208084 79.375) (end 94.242606 80.40952) (width 0.25) (layer "F.Cu") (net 3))
 (segment (start 84.013928 78.74) (end 84.648928 79.375) (width 0.25) (layer "F.Cu") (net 3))
 (segment (start 94.242606 80.40952) (end 96.213092 80.40952) (width 0.25) (layer "F.Cu") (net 3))
 (segment (start 100.965 87.684022) (end 102.180978 88.9) (width 0.25) (layer "F.Cu") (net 3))
 (segment (start 102.61 88.9) (end 102.61 90.17) (width 0.25) (layer "F.Cu") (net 3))
 (segment (start 96.213092 80.40952) (end 100.965 85.161428) (width 0.25) (layer "F.Cu") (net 3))
 (segment (start 102.180978 88.9) (end 102.61 88.9) (width 0.25) (layer "F.Cu") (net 3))
 (segment (start 83.25 78.74) (end 84.013928 78.74) (width 0.25) (layer "F.Cu") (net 3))
 (segment (start 100.965 85.161428) (end 100.965 87.684022) (width 0.25) (layer "F.Cu") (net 3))
 (segment (start 88.2 78.74) (end 93.208802 78.74) (width 0.25) (layer "F.Cu") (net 13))
 (segment (start 101.485489 84.975489) (end 101.485489 85.764511) (width 0.35) (layer "F.Cu") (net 13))
 (segment (start 94.428803 79.96) (end 96.47 79.96) (width 0.25) (layer "F.Cu") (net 13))
 (segment (start 93.208802 78.74) (end 94.428803 79.96) (width 0.25) (layer "F.Cu") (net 13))
 (segment (start 96.47 79.96) (end 101.485489 84.975489) (width 0.25) (layer "F.Cu") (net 13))
 (segment (start 101.485489 85.764511) (end 102.080978 86.36) (width 0.35) (layer "F.Cu") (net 13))
 (segment (start 102.61 86.36) (end 102.61 87.63) (width 0.25) (layer "F.Cu") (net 13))
 (segment (start 93.19904 78.09452) (end 94.615 79.51048) (width 0.25) (layer "F.Cu") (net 2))
 (segment (start 94.615 79.51048) (end 97.85048 79.51048) (width 0.25) (layer "F.Cu") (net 2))
 (segment (start 83.25 77.47) (end 83.87452 78.09452) (width 0.25) (layer "F.Cu") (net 2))
 (segment (start 102.61 83.82) (end 102.61 85.09) (width 0.25) (layer "F.Cu") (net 2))
 (segment (start 102.16 83.82) (end 102.61 83.82) (width 0.25) (layer "F.Cu") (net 2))
 (segment (start 97.85048 79.51048) (end 102.16 83.82) (width 0.25) (layer "F.Cu") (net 2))
 (segment (start 83.87452 78.09452) (end 93.19904 78.09452) (width 0.25) (layer "F.Cu") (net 2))
 (segment (start 102.87 82.55) (end 102.61 82.55) (width 0.35) (layer "F.Cu") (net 14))
 (segment (start 93.499022 77.47) (end 94.769022 78.74) (width 0.35) (layer "F.Cu") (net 14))
 (segment (start 88.2 77.47) (end 93.499022 77.47) (width 0.35) (layer "F.Cu") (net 14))
 (segment (start 99.695 78.74) (end 102.61 81.655) (width 0.35) (layer "F.Cu") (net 14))
 (segment (start 102.61 82.29) (end 102.87 82.55) (width 0.35) (layer "F.Cu") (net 14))
 (segment (start 102.61 81.28) (end 102.61 82.29) (width 0.35) (layer "F.Cu") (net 14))
 (segment (start 102.61 81.655) (end 102.61 82.55) (width 0.35) (layer "F.Cu") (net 14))
 (segment (start 94.769022 78.74) (end 99.695 78.74) (width 0.35) (layer "F.Cu") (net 14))
 (segment (start 86.1 90.6) (end 84.75 90.6) (width 0.25) (layer "F.Cu") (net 25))
 (segment (start 85.95 91.55) (end 84.75 91.55) (width 0.25) (layer "F.Cu") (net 25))
 (segment (start 86.5 91) (end 85.95 91.55) (width 0.25) (layer "F.Cu") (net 25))
 (segment (start 84.455 106.68) (end 85.07 106.065) (width 0.25) (layer "F.Cu") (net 25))
 (segment (start 85.07 95.33) (end 85.07 99.06) (width 0.25) (layer "F.Cu") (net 25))
 (segment (start 85.07 99.06) (end 88.25 99.06) (width 0.25) (layer "F.Cu") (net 25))
 (segment (start 85.07 106.065) (end 85.07 99.06) (width 0.25) (layer "F.Cu") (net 25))
 (segment (start 86.5 91) (end 86.1 90.6) (width 0.25) (layer "F.Cu") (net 25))
 (segment (start 86.1 94.3) (end 85.07 95.33) (width 0.25) (layer "F.Cu") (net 25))
 (via (at 86.5 91) (size 0.8) (drill 0.4) (layers "F.Cu" "B.Cu") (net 25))
 (via (at 86.1 94.3) (size 0.8) (drill 0.4) (layers "F.Cu" "B.Cu") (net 25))
 (segment (start 86.5 93.9) (end 86.1 94.3) (width 0.25) (layer "B.Cu") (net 25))
 (segment (start 86.5 91) (end 86.5 93.9) (width 0.25) (layer "B.Cu") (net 25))
 (segment (start 90.805 83.82) (end 92.71 81.915) (width 0.25) (layer "F.Cu") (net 10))
 (segment (start 88.2 83.82) (end 90.805 83.82) (width 0.25) (layer "F.Cu") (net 10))
 (via (at 92.71 81.915) (size 0.8) (drill 0.4) (layers "F.Cu" "B.Cu") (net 10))
 (segment (start 92.71 81.915) (end 95.25 81.915) (width 0.25) (layer "B.Cu") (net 10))
 (segment (start 95.25 81.915) (end 105.41 71.755) (width 0.25) (layer "B.Cu") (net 10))
 (segment (start 92.71 80.0995) (end 92.6205 80.01) (width 0.25) (layer "F.Cu") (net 12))
 (segment (start 92.6205 80.01) (end 88.2 80.01) (width 0.25) (layer "F.Cu") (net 12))
 (via (at 92.71 80.0995) (size 0.8) (drill 0.4) (layers "F.Cu" "B.Cu") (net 12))
 (segment (start 92.71 80.0995) (end 94.5255 80.0995) (width 0.25) (layer "B.Cu") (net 12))
 (segment (start 94.5255 80.0995) (end 102.87 71.755) (width 0.25) (layer "B.Cu") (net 12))
 (segment (start 88.2 81.28) (end 90.805 81.28) (width 0.25) (layer "F.Cu") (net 11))
 (via (at 90.805 81.28) (size 0.8) (drill 0.4) (layers "F.Cu" "B.Cu") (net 11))
 (segment (start 90.805 81.28) (end 90.805 80.979886) (width 0.25) (layer "B.Cu") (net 11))
 (segment (start 100.029886 71.755) (end 100.33 71.755) (width 0.25) (layer "B.Cu") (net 11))
 (segment (start 90.805 80.979886) (end 100.029886 71.755) (width 0.25) (layer "B.Cu") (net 11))
 (segment (start 110.115 80.385) (end 108.83 80.385) (width 0.25) (layer "F.Cu") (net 16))
 (segment (start 97.155 73.66) (end 110.49 73.66) (width 0.25) (layer "F.Cu") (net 16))
 (segment (start 95.25 71.755) (end 97.155 73.66) (width 0.25) (layer "F.Cu") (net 16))
 (segment (start 111.125 79.375) (end 110.115 80.385) (width 0.25) (layer "F.Cu") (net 16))
 (segment (start 110.49 73.66) (end 111.125 74.295) (width 0.25) (layer "F.Cu") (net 16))
 (segment (start 111.125 74.295) (end 111.125 79.375) (width 0.25) (layer "F.Cu") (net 16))
 (segment (start 111.76 103.505) (end 114.935 106.68) (width 0.25) (layer "F.Cu") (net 22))
 (segment (start 111.76 99.69) (end 111.76 103.505) (width 0.25) (layer "F.Cu") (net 22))
 (segment (start 98.45 95.8) (end 98.45 96.75) (width 0.25) (layer "F.Cu") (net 22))
 (segment (start 82.25 89.65) (end 83.3 88.6) (width 0.25) (layer "F.Cu") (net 23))
 (segment (start 90.83 90.17) (end 95.51 90.17) (width 0.25) (layer "F.Cu") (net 23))
 (segment (start 83.3 88.6) (end 89.2 88.6) (width 0.25) (layer "F.Cu") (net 23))
 (segment (start 90.8 90.2) (end 90.83 90.17) (width 0.25) (layer "F.Cu") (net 23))
 (segment (start 89.2 88.6) (end 90.8 90.2) (width 0.25) (layer "F.Cu") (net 23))
 (segment (start 82.2 91.5) (end 82.25 91.55) (width 0.25) (layer "F.Cu") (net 24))
 (segment (start 82.44 86.36) (end 81.8 87) (width 0.25) (layer "F.Cu") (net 24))
 (segment (start 95.51 86.36) (end 82.44 86.36) (width 0.25) (layer "F.Cu") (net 24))
 (segment (start 80.5 91.5) (end 82.2 91.5) (width 0.25) (layer "F.Cu") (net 24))
 (via (at 80.5 91.5) (size 0.8) (drill 0.4) (layers "F.Cu" "B.Cu") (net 24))
 (via (at 81.8 87) (size 0.8) (drill 0.4) (layers "F.Cu" "B.Cu") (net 24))
 (segment (start 81.8 87) (end 80.5 88.3) (width 0.25) (layer "B.Cu") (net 24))
 (segment (start 80.5 88.3) (end 80.5 91.5) (width 0.25) (layer "B.Cu") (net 24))
 (segment (start 88.95 92.05) (end 88.95 90.75) (width 0.25) (layer "F.Cu") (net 20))
 (segment (start 88.95 90.75) (end 89 90.7) (width 0.25) (layer "F.Cu") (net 20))
 (segment (start 91.1 88.9) (end 95.51 88.9) (width 0.25) (layer "F.Cu") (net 20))
 (via (at 91.1 88.9) (size 0.8) (drill 0.4) (layers "F.Cu" "B.Cu") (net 20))
 (via (at 89 90.7) (size 0.8) (drill 0.4) (layers "F.Cu" "B.Cu") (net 20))
 (segment (start 90.8 88.9) (end 91.1 88.9) (width 0.25) (layer "B.Cu") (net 20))
 (segment (start 89 90.7) (end 90.8 88.9) (width 0.25) (layer "B.Cu") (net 20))
 (segment (start 88.95 94.95) (end 89.4 95.4) (width 0.25) (layer "F.Cu") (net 21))
 (segment (start 92.5 87.6) (end 92.53 87.63) (width 0.25) (layer "F.Cu") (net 21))
 (segment (start 88.95 93.95) (end 88.95 94.95) (width 0.25) (layer "F.Cu") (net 21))
 (segment (start 95.51 87.63) (end 95.96 87.63) (width 0.25) (layer "F.Cu") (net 21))
 (segment (start 92.53 87.63) (end 95.51 87.63) (width 0.25) (layer "F.Cu") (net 21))
 (via (at 89.4 95.4) (size 0.8) (drill 0.4) (layers "F.Cu" "B.Cu") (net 21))
 (via (at 92.5 87.6) (size 0.8) (drill 0.4) (layers "F.Cu" "B.Cu") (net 21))
 (segment (start 89.4 95.4) (end 92.4 92.4) (width 0.25) (layer "B.Cu") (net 21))
 (segment (start 92.4 87.7) (end 92.5 87.6) (width 0.25) (layer "B.Cu") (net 21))
 (segment (start 92.4 92.4) (end 92.4 87.7) (width 0.25) (layer "B.Cu") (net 21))
 (segment (start 95.51 85.09) (end 95.939022 85.09) (width 0.25) (layer "F.Cu") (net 29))
 (segment (start 95.939022 85.09) (end 98.425 87.575978) (width 0.25) (layer "F.Cu") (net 29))
 (segment (start 95.51 81.28) (end 95.96 81.28) (width 0.25) (layer "F.Cu") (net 26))
 (segment (start 95.96 81.28) (end 100.51548 85.83548) (width 0.25) (layer "F.Cu") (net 26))
 (segment (start 95.96 82.55) (end 100.06596 86.65596) (width 0.25) (layer "F.Cu") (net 27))
 (segment (start 95.51 82.55) (end 95.96 82.55) (width 0.25) (layer "F.Cu") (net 27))
 (segment (start 96.155489 84.465489) (end 96.584511 84.465489) (width 0.25) (layer "F.Cu") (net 28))
 (segment (start 95.51 83.82) (end 96.155489 84.465489) (width 0.25) (layer "F.Cu") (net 28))
 (segment (start 96.584511 84.465489) (end 99.06 86.940978) (width 0.25) (layer "F.Cu") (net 28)))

